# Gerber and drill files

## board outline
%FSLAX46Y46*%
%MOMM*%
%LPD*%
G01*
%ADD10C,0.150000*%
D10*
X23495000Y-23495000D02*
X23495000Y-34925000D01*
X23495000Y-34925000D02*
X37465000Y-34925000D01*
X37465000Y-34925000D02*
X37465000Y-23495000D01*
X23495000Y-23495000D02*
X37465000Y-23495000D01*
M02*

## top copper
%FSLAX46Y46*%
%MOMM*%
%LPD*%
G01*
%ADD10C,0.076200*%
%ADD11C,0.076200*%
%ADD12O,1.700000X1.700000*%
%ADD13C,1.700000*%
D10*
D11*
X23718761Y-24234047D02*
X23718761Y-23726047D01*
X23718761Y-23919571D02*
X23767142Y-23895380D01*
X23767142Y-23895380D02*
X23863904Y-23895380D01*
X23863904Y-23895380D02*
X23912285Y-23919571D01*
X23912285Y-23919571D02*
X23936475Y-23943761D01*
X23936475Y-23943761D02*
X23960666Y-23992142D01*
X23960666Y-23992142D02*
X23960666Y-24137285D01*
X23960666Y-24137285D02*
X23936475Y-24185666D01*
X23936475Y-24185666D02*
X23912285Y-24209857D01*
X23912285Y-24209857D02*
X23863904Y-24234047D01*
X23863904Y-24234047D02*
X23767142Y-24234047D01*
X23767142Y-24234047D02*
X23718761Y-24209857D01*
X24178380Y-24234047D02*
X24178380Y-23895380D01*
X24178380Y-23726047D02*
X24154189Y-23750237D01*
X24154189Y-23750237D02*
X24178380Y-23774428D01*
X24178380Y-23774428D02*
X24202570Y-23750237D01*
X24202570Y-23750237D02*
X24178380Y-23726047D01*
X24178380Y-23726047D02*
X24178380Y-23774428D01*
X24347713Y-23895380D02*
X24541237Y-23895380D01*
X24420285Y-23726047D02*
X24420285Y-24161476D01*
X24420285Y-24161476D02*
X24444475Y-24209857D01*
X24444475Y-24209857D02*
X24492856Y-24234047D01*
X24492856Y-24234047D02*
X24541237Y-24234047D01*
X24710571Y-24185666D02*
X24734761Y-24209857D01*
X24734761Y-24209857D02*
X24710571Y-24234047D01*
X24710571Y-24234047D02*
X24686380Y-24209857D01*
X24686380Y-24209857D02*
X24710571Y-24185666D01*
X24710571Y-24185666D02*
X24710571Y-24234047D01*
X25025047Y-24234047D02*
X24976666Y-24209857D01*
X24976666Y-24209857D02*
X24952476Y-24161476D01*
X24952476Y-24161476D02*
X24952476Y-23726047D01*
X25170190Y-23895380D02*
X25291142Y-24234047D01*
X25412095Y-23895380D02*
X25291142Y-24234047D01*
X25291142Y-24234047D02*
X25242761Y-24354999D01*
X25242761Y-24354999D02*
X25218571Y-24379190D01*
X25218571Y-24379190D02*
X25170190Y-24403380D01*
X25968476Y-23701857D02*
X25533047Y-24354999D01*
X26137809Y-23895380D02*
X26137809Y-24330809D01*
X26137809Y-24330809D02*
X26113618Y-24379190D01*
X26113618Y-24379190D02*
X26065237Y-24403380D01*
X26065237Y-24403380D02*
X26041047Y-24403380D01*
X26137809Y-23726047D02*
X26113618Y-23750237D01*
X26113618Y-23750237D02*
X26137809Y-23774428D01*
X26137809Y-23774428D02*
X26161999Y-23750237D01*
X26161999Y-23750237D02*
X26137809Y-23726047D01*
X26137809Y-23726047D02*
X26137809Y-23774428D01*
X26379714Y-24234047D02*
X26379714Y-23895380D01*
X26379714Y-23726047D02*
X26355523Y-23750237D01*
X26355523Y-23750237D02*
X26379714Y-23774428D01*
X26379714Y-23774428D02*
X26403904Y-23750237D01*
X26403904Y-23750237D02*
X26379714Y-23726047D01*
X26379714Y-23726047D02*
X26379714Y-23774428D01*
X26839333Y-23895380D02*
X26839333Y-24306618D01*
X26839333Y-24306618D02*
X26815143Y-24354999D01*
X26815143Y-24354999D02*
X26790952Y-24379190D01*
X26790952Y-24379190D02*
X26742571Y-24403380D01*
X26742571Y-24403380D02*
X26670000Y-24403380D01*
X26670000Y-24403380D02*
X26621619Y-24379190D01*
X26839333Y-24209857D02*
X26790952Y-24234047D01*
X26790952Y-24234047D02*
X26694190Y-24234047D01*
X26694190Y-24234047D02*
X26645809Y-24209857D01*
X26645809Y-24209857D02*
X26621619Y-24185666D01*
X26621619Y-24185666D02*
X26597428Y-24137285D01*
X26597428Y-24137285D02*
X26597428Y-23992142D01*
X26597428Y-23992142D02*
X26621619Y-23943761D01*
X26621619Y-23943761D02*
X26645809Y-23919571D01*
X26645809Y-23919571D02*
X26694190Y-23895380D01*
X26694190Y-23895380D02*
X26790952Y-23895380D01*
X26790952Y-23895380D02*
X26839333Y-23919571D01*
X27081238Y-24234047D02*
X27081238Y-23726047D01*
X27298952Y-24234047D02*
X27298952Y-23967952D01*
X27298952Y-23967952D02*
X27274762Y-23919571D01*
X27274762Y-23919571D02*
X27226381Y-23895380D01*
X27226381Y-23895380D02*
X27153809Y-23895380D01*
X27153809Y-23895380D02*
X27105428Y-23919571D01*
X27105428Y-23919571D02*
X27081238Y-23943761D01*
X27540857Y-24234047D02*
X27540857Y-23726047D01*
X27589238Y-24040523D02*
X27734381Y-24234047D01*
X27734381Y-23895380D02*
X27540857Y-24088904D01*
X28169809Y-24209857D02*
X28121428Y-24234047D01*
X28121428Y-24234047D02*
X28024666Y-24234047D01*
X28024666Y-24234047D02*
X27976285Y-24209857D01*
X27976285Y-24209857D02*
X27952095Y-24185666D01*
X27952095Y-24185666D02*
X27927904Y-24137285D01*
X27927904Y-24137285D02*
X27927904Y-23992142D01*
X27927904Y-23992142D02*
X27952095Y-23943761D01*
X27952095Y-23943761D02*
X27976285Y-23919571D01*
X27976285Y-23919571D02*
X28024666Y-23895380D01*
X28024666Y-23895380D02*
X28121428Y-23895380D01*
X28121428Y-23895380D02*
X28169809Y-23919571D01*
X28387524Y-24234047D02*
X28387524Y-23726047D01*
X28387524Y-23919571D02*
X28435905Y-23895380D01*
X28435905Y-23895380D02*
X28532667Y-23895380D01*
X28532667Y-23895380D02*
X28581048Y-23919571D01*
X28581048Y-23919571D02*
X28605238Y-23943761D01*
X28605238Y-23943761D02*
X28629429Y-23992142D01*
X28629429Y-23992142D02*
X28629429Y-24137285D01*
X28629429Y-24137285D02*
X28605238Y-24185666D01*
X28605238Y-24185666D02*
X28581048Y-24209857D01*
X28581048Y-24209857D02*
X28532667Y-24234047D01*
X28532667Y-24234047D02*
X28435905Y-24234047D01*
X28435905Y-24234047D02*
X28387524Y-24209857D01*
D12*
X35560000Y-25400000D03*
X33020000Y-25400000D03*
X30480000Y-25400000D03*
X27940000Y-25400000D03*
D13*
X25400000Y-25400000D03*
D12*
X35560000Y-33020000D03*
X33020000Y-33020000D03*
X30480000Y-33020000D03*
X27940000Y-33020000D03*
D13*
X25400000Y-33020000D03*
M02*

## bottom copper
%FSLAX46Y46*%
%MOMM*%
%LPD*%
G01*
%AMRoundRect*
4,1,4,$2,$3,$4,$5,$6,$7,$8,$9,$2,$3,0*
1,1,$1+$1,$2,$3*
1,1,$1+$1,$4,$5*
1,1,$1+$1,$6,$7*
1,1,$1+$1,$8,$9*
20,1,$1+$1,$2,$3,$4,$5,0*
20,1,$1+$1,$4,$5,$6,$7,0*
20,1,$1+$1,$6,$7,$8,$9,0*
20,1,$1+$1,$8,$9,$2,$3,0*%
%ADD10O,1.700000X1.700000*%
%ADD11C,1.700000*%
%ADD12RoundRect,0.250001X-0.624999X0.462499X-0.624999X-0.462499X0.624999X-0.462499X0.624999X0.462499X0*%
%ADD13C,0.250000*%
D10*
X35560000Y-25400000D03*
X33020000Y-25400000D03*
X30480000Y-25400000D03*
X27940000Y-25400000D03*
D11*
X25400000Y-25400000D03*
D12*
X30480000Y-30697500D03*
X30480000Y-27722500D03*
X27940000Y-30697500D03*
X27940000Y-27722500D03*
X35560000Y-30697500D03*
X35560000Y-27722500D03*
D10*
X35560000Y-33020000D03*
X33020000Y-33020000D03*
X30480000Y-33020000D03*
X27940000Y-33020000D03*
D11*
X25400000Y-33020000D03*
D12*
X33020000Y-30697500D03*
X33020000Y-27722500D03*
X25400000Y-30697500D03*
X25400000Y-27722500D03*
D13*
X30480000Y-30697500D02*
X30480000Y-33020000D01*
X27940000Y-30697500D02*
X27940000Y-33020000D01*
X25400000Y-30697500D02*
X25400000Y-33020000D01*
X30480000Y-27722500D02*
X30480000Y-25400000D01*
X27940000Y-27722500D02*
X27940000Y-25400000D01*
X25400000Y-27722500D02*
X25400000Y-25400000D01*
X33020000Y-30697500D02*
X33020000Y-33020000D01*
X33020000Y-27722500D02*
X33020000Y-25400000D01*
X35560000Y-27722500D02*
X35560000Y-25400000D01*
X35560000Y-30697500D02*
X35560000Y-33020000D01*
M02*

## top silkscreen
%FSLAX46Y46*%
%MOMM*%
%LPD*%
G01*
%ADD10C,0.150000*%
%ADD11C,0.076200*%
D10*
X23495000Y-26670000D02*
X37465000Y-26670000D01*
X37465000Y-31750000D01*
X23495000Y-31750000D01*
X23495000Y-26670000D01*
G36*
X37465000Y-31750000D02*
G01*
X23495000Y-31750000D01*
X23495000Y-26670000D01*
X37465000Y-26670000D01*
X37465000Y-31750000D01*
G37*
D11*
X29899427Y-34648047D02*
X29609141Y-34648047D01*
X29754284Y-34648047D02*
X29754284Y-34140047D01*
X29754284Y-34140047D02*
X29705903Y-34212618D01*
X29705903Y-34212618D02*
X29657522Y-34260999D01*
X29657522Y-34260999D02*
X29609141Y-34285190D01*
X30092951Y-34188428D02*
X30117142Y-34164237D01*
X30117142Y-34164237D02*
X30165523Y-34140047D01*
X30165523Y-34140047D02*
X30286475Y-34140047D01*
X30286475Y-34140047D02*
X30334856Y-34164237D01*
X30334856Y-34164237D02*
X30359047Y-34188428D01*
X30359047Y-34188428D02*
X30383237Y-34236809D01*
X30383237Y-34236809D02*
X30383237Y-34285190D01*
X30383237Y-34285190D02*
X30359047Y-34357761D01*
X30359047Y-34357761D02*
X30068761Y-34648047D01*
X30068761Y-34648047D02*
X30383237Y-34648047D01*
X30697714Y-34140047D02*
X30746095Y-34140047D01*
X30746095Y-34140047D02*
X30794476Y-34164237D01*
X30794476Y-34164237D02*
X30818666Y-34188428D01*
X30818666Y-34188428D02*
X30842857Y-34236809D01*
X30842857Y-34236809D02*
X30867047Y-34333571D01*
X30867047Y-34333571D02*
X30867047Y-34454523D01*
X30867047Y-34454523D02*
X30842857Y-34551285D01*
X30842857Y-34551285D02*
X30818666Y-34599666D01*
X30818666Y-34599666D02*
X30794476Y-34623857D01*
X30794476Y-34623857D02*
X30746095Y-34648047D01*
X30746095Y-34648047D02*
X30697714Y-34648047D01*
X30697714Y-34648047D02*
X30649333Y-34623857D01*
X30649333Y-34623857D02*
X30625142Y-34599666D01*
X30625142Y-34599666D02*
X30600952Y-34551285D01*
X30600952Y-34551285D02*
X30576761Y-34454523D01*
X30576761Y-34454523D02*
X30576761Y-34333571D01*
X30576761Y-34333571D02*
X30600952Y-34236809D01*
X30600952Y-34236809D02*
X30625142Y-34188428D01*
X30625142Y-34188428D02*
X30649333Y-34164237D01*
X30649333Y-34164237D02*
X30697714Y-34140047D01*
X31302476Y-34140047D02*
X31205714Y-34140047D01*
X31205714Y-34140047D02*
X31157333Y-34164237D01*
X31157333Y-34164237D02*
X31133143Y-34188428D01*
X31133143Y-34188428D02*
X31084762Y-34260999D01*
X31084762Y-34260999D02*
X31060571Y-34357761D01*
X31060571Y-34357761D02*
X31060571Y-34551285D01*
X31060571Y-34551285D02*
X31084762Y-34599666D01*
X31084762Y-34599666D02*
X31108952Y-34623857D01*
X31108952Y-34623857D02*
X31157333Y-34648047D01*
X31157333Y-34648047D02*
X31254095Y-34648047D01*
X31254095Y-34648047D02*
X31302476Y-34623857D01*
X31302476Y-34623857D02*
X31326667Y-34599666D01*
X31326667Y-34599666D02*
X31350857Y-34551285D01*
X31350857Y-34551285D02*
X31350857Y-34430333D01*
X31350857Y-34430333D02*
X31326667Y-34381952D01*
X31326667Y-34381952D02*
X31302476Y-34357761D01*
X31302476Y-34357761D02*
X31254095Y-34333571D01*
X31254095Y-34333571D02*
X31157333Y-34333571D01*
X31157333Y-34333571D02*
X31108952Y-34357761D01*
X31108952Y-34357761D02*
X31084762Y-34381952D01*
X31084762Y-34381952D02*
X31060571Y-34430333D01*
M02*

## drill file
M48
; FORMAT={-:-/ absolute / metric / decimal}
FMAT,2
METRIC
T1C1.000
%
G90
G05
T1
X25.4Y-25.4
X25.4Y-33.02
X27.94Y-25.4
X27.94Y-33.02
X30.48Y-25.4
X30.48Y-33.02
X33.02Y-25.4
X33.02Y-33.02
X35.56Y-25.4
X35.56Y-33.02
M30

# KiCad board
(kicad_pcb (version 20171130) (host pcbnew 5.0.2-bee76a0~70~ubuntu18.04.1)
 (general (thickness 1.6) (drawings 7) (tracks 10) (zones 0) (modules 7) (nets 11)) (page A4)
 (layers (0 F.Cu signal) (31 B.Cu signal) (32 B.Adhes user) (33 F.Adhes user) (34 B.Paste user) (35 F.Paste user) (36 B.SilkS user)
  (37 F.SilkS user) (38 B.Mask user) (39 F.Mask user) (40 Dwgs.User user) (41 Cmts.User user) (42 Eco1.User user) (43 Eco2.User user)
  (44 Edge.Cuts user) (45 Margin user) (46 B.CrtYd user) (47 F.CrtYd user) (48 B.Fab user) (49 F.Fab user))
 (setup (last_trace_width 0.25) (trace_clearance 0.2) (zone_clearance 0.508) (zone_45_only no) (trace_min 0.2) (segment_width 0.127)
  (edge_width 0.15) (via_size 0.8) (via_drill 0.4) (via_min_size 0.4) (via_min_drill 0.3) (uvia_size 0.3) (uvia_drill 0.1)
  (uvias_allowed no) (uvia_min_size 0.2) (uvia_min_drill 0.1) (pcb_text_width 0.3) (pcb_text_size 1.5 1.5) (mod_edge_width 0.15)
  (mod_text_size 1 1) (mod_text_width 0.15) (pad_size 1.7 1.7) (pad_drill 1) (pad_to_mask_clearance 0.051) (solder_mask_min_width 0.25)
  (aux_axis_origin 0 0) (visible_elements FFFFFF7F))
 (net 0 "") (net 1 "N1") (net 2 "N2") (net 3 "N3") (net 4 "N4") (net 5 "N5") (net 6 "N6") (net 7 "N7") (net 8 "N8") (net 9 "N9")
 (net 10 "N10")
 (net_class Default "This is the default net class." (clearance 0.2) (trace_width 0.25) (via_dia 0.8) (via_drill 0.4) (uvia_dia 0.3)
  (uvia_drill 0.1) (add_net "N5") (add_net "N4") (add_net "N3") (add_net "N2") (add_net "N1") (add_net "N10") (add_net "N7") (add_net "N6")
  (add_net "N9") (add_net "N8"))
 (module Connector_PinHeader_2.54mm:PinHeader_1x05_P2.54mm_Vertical (layer B.Cu) (at 25.4 25.4 270)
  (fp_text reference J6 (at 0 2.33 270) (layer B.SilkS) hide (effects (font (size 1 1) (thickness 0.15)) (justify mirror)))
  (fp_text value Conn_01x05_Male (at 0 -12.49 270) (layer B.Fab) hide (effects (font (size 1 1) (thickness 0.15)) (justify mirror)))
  (pad 5 thru_hole oval (at 0 -10.16 270) (size 1.7 1.7) (drill 1) (layers *.Cu *.Mask) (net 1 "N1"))
  (pad 4 thru_hole oval (at 0 -7.62 270) (size 1.7 1.7) (drill 1) (layers *.Cu *.Mask) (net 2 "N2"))
  (pad 3 thru_hole oval (at 0 -5.08 270) (size 1.7 1.7) (drill 1) (layers *.Cu *.Mask) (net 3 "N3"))
  (pad 2 thru_hole oval (at 0 -2.54 270) (size 1.7 1.7) (drill 1) (layers *.Cu *.Mask) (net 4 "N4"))
  (pad 1 thru_hole circle (at 0 0 270) (size 1.7 1.7) (drill 1) (layers *.Cu *.Mask) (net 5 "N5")))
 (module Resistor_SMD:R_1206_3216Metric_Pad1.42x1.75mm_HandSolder (layer B.Cu) (at 30.48 29.21 270)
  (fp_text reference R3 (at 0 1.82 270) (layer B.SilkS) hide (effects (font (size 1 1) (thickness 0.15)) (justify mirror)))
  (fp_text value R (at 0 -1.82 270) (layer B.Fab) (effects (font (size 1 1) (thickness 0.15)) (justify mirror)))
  (pad 2 smd roundrect (at 1.4875 0 270) (size 1.425 1.75) (layers B.Cu B.Paste B.Mask) (roundrect_rratio 0.175439) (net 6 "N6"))
  (pad 1 smd roundrect (at -1.4875 0 270) (size 1.425 1.75) (layers B.Cu B.Paste B.Mask) (roundrect_rratio 0.175439) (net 3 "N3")))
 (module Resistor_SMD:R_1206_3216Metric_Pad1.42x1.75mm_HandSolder (layer B.Cu) (at 27.94 29.21 270)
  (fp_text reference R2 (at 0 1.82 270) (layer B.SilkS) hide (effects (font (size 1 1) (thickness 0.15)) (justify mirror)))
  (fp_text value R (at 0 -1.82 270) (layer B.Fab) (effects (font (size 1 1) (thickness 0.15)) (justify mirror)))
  (pad 2 smd roundrect (at 1.4875 0 270) (size 1.425 1.75) (layers B.Cu B.Paste B.Mask) (roundrect_rratio 0.175439) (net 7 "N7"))
  (pad 1 smd roundrect (at -1.4875 0 270) (size 1.425 1.75) (layers B.Cu B.Paste B.Mask) (roundrect_rratio 0.175439) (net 4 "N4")))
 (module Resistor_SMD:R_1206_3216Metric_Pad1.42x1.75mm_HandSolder (layer B.Cu) (at 35.56 29.21 270)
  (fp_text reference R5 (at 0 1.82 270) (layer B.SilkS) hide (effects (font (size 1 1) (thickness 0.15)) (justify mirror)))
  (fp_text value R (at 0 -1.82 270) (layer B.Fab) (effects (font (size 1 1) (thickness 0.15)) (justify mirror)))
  (pad 2 smd roundrect (at 1.4875 0 270) (size 1.425 1.75) (layers B.Cu B.Paste B.Mask) (roundrect_rratio 0.175439) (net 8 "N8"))
  (pad 1 smd roundrect (at -1.4875 0 270) (size 1.425 1.75) (layers B.Cu B.Paste B.Mask) (roundrect_rratio 0.175439) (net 1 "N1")))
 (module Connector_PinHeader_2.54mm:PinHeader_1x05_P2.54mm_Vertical (layer B.Cu) (at 25.4 33.02 270)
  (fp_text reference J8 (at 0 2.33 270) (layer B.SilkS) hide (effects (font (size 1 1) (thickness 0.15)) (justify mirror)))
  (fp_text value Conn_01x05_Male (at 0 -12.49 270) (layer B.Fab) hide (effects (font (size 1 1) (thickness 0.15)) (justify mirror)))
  (pad 5 thru_hole oval (at 0 -10.16 270) (size 1.7 1.7) (drill 1) (layers *.Cu *.Mask) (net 8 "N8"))
  (pad 4 thru_hole oval (at 0 -7.62 270) (size 1.7 1.7) (drill 1) (layers *.Cu *.Mask) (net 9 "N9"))
  (pad 3 thru_hole oval (at 0 -5.08 270) (size 1.7 1.7) (drill 1) (layers *.Cu *.Mask) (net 6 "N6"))
  (pad 2 thru_hole oval (at 0 -2.54 270) (size 1.7 1.7) (drill 1) (layers *.Cu *.Mask) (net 7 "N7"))
  (pad 1 thru_hole circle (at 0 0 270) (size 1.7 1.7) (drill 1) (layers *.Cu *.Mask) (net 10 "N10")))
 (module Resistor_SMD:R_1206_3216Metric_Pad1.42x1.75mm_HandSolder (layer B.Cu) (at 33.02 29.21 270)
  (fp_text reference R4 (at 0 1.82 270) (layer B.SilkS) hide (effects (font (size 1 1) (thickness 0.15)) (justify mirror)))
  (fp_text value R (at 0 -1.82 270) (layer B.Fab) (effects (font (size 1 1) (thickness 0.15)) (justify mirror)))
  (pad 2 smd roundrect (at 1.4875 0 270) (size 1.425 1.75) (layers B.Cu B.Paste B.Mask) (roundrect_rratio 0.175439) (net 9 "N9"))
  (pad 1 smd roundrect (at -1.4875 0 270) (size 1.425 1.75) (layers B.Cu B.Paste B.Mask) (roundrect_rratio 0.175439) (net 2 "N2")))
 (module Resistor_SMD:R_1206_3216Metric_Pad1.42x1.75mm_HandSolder (layer B.Cu) (at 25.4 29.21 270)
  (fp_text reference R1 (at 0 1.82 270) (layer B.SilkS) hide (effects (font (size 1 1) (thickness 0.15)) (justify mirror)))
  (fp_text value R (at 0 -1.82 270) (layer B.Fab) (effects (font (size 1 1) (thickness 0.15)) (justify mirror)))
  (pad 2 smd roundrect (at 1.4875 0 270) (size 1.425 1.75) (layers B.Cu B.Paste B.Mask) (roundrect_rratio 0.175439) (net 10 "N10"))
  (pad 1 smd roundrect (at -1.4875 0 270) (size 1.425 1.75) (layers B.Cu B.Paste B.Mask) (roundrect_rratio 0.175439) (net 5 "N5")))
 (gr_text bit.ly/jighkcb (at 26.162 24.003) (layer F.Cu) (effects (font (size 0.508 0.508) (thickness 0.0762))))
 (gr_poly (pts (xy 23.495 26.67) (xy 37.465 26.67) (xy 37.465 31.75) (xy 23.495 31.75)) (layer F.SilkS) (width 0.15))
 (gr_line (start 23.495 23.495) (end 23.495 34.925) (layer Edge.Cuts) (width 0.15))
 (gr_line (start 23.495 34.925) (end 37.465 34.925) (layer Edge.Cuts) (width 0.15))
 (gr_line (start 37.465 34.925) (end 37.465 23.495) (layer Edge.Cuts) (width 0.15))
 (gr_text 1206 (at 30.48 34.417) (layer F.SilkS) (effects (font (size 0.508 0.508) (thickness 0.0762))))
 (gr_line (start 23.495 23.495) (end 37.465 23.495) (layer Edge.Cuts) (width 0.15))
 (segment (start 30.48 30.6975) (end 30.48 33.02) (width 0.25) (layer B.Cu) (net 6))
 (segment (start 27.94 30.6975) (end 27.94 33.02) (width 0.25) (layer B.Cu) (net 7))
 (segment (start 25.4 30.6975) (end 25.4 33.02) (width 0.25) (layer B.Cu) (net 10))
 (segment (start 30.48 27.7225) (end 30.48 25.4) (width 0.25) (layer B.Cu) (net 3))
 (segment (start 27.94 27.7225) (end 27.94 25.4) (width 0.25) (layer B.Cu) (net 4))
 (segment (start 25.4 27.7225) (end 25.4 25.4) (width 0.25) (layer B.Cu) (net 5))
 (segment (start 33.02 30.6975) (end 33.02 33.02) (width 0.25) (layer B.Cu) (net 9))
 (segment (start 33.02 27.7225) (end 33.02 25.4) (width 0.25) (layer B.Cu) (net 2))
 (segment (start 35.56 27.7225) (end 35.56 25.4) (width 0.25) (layer B.Cu) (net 1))
 (segment (start 35.56 30.6975) (end 35.56 33.02) (width 0.25) (layer B.Cu) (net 8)))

